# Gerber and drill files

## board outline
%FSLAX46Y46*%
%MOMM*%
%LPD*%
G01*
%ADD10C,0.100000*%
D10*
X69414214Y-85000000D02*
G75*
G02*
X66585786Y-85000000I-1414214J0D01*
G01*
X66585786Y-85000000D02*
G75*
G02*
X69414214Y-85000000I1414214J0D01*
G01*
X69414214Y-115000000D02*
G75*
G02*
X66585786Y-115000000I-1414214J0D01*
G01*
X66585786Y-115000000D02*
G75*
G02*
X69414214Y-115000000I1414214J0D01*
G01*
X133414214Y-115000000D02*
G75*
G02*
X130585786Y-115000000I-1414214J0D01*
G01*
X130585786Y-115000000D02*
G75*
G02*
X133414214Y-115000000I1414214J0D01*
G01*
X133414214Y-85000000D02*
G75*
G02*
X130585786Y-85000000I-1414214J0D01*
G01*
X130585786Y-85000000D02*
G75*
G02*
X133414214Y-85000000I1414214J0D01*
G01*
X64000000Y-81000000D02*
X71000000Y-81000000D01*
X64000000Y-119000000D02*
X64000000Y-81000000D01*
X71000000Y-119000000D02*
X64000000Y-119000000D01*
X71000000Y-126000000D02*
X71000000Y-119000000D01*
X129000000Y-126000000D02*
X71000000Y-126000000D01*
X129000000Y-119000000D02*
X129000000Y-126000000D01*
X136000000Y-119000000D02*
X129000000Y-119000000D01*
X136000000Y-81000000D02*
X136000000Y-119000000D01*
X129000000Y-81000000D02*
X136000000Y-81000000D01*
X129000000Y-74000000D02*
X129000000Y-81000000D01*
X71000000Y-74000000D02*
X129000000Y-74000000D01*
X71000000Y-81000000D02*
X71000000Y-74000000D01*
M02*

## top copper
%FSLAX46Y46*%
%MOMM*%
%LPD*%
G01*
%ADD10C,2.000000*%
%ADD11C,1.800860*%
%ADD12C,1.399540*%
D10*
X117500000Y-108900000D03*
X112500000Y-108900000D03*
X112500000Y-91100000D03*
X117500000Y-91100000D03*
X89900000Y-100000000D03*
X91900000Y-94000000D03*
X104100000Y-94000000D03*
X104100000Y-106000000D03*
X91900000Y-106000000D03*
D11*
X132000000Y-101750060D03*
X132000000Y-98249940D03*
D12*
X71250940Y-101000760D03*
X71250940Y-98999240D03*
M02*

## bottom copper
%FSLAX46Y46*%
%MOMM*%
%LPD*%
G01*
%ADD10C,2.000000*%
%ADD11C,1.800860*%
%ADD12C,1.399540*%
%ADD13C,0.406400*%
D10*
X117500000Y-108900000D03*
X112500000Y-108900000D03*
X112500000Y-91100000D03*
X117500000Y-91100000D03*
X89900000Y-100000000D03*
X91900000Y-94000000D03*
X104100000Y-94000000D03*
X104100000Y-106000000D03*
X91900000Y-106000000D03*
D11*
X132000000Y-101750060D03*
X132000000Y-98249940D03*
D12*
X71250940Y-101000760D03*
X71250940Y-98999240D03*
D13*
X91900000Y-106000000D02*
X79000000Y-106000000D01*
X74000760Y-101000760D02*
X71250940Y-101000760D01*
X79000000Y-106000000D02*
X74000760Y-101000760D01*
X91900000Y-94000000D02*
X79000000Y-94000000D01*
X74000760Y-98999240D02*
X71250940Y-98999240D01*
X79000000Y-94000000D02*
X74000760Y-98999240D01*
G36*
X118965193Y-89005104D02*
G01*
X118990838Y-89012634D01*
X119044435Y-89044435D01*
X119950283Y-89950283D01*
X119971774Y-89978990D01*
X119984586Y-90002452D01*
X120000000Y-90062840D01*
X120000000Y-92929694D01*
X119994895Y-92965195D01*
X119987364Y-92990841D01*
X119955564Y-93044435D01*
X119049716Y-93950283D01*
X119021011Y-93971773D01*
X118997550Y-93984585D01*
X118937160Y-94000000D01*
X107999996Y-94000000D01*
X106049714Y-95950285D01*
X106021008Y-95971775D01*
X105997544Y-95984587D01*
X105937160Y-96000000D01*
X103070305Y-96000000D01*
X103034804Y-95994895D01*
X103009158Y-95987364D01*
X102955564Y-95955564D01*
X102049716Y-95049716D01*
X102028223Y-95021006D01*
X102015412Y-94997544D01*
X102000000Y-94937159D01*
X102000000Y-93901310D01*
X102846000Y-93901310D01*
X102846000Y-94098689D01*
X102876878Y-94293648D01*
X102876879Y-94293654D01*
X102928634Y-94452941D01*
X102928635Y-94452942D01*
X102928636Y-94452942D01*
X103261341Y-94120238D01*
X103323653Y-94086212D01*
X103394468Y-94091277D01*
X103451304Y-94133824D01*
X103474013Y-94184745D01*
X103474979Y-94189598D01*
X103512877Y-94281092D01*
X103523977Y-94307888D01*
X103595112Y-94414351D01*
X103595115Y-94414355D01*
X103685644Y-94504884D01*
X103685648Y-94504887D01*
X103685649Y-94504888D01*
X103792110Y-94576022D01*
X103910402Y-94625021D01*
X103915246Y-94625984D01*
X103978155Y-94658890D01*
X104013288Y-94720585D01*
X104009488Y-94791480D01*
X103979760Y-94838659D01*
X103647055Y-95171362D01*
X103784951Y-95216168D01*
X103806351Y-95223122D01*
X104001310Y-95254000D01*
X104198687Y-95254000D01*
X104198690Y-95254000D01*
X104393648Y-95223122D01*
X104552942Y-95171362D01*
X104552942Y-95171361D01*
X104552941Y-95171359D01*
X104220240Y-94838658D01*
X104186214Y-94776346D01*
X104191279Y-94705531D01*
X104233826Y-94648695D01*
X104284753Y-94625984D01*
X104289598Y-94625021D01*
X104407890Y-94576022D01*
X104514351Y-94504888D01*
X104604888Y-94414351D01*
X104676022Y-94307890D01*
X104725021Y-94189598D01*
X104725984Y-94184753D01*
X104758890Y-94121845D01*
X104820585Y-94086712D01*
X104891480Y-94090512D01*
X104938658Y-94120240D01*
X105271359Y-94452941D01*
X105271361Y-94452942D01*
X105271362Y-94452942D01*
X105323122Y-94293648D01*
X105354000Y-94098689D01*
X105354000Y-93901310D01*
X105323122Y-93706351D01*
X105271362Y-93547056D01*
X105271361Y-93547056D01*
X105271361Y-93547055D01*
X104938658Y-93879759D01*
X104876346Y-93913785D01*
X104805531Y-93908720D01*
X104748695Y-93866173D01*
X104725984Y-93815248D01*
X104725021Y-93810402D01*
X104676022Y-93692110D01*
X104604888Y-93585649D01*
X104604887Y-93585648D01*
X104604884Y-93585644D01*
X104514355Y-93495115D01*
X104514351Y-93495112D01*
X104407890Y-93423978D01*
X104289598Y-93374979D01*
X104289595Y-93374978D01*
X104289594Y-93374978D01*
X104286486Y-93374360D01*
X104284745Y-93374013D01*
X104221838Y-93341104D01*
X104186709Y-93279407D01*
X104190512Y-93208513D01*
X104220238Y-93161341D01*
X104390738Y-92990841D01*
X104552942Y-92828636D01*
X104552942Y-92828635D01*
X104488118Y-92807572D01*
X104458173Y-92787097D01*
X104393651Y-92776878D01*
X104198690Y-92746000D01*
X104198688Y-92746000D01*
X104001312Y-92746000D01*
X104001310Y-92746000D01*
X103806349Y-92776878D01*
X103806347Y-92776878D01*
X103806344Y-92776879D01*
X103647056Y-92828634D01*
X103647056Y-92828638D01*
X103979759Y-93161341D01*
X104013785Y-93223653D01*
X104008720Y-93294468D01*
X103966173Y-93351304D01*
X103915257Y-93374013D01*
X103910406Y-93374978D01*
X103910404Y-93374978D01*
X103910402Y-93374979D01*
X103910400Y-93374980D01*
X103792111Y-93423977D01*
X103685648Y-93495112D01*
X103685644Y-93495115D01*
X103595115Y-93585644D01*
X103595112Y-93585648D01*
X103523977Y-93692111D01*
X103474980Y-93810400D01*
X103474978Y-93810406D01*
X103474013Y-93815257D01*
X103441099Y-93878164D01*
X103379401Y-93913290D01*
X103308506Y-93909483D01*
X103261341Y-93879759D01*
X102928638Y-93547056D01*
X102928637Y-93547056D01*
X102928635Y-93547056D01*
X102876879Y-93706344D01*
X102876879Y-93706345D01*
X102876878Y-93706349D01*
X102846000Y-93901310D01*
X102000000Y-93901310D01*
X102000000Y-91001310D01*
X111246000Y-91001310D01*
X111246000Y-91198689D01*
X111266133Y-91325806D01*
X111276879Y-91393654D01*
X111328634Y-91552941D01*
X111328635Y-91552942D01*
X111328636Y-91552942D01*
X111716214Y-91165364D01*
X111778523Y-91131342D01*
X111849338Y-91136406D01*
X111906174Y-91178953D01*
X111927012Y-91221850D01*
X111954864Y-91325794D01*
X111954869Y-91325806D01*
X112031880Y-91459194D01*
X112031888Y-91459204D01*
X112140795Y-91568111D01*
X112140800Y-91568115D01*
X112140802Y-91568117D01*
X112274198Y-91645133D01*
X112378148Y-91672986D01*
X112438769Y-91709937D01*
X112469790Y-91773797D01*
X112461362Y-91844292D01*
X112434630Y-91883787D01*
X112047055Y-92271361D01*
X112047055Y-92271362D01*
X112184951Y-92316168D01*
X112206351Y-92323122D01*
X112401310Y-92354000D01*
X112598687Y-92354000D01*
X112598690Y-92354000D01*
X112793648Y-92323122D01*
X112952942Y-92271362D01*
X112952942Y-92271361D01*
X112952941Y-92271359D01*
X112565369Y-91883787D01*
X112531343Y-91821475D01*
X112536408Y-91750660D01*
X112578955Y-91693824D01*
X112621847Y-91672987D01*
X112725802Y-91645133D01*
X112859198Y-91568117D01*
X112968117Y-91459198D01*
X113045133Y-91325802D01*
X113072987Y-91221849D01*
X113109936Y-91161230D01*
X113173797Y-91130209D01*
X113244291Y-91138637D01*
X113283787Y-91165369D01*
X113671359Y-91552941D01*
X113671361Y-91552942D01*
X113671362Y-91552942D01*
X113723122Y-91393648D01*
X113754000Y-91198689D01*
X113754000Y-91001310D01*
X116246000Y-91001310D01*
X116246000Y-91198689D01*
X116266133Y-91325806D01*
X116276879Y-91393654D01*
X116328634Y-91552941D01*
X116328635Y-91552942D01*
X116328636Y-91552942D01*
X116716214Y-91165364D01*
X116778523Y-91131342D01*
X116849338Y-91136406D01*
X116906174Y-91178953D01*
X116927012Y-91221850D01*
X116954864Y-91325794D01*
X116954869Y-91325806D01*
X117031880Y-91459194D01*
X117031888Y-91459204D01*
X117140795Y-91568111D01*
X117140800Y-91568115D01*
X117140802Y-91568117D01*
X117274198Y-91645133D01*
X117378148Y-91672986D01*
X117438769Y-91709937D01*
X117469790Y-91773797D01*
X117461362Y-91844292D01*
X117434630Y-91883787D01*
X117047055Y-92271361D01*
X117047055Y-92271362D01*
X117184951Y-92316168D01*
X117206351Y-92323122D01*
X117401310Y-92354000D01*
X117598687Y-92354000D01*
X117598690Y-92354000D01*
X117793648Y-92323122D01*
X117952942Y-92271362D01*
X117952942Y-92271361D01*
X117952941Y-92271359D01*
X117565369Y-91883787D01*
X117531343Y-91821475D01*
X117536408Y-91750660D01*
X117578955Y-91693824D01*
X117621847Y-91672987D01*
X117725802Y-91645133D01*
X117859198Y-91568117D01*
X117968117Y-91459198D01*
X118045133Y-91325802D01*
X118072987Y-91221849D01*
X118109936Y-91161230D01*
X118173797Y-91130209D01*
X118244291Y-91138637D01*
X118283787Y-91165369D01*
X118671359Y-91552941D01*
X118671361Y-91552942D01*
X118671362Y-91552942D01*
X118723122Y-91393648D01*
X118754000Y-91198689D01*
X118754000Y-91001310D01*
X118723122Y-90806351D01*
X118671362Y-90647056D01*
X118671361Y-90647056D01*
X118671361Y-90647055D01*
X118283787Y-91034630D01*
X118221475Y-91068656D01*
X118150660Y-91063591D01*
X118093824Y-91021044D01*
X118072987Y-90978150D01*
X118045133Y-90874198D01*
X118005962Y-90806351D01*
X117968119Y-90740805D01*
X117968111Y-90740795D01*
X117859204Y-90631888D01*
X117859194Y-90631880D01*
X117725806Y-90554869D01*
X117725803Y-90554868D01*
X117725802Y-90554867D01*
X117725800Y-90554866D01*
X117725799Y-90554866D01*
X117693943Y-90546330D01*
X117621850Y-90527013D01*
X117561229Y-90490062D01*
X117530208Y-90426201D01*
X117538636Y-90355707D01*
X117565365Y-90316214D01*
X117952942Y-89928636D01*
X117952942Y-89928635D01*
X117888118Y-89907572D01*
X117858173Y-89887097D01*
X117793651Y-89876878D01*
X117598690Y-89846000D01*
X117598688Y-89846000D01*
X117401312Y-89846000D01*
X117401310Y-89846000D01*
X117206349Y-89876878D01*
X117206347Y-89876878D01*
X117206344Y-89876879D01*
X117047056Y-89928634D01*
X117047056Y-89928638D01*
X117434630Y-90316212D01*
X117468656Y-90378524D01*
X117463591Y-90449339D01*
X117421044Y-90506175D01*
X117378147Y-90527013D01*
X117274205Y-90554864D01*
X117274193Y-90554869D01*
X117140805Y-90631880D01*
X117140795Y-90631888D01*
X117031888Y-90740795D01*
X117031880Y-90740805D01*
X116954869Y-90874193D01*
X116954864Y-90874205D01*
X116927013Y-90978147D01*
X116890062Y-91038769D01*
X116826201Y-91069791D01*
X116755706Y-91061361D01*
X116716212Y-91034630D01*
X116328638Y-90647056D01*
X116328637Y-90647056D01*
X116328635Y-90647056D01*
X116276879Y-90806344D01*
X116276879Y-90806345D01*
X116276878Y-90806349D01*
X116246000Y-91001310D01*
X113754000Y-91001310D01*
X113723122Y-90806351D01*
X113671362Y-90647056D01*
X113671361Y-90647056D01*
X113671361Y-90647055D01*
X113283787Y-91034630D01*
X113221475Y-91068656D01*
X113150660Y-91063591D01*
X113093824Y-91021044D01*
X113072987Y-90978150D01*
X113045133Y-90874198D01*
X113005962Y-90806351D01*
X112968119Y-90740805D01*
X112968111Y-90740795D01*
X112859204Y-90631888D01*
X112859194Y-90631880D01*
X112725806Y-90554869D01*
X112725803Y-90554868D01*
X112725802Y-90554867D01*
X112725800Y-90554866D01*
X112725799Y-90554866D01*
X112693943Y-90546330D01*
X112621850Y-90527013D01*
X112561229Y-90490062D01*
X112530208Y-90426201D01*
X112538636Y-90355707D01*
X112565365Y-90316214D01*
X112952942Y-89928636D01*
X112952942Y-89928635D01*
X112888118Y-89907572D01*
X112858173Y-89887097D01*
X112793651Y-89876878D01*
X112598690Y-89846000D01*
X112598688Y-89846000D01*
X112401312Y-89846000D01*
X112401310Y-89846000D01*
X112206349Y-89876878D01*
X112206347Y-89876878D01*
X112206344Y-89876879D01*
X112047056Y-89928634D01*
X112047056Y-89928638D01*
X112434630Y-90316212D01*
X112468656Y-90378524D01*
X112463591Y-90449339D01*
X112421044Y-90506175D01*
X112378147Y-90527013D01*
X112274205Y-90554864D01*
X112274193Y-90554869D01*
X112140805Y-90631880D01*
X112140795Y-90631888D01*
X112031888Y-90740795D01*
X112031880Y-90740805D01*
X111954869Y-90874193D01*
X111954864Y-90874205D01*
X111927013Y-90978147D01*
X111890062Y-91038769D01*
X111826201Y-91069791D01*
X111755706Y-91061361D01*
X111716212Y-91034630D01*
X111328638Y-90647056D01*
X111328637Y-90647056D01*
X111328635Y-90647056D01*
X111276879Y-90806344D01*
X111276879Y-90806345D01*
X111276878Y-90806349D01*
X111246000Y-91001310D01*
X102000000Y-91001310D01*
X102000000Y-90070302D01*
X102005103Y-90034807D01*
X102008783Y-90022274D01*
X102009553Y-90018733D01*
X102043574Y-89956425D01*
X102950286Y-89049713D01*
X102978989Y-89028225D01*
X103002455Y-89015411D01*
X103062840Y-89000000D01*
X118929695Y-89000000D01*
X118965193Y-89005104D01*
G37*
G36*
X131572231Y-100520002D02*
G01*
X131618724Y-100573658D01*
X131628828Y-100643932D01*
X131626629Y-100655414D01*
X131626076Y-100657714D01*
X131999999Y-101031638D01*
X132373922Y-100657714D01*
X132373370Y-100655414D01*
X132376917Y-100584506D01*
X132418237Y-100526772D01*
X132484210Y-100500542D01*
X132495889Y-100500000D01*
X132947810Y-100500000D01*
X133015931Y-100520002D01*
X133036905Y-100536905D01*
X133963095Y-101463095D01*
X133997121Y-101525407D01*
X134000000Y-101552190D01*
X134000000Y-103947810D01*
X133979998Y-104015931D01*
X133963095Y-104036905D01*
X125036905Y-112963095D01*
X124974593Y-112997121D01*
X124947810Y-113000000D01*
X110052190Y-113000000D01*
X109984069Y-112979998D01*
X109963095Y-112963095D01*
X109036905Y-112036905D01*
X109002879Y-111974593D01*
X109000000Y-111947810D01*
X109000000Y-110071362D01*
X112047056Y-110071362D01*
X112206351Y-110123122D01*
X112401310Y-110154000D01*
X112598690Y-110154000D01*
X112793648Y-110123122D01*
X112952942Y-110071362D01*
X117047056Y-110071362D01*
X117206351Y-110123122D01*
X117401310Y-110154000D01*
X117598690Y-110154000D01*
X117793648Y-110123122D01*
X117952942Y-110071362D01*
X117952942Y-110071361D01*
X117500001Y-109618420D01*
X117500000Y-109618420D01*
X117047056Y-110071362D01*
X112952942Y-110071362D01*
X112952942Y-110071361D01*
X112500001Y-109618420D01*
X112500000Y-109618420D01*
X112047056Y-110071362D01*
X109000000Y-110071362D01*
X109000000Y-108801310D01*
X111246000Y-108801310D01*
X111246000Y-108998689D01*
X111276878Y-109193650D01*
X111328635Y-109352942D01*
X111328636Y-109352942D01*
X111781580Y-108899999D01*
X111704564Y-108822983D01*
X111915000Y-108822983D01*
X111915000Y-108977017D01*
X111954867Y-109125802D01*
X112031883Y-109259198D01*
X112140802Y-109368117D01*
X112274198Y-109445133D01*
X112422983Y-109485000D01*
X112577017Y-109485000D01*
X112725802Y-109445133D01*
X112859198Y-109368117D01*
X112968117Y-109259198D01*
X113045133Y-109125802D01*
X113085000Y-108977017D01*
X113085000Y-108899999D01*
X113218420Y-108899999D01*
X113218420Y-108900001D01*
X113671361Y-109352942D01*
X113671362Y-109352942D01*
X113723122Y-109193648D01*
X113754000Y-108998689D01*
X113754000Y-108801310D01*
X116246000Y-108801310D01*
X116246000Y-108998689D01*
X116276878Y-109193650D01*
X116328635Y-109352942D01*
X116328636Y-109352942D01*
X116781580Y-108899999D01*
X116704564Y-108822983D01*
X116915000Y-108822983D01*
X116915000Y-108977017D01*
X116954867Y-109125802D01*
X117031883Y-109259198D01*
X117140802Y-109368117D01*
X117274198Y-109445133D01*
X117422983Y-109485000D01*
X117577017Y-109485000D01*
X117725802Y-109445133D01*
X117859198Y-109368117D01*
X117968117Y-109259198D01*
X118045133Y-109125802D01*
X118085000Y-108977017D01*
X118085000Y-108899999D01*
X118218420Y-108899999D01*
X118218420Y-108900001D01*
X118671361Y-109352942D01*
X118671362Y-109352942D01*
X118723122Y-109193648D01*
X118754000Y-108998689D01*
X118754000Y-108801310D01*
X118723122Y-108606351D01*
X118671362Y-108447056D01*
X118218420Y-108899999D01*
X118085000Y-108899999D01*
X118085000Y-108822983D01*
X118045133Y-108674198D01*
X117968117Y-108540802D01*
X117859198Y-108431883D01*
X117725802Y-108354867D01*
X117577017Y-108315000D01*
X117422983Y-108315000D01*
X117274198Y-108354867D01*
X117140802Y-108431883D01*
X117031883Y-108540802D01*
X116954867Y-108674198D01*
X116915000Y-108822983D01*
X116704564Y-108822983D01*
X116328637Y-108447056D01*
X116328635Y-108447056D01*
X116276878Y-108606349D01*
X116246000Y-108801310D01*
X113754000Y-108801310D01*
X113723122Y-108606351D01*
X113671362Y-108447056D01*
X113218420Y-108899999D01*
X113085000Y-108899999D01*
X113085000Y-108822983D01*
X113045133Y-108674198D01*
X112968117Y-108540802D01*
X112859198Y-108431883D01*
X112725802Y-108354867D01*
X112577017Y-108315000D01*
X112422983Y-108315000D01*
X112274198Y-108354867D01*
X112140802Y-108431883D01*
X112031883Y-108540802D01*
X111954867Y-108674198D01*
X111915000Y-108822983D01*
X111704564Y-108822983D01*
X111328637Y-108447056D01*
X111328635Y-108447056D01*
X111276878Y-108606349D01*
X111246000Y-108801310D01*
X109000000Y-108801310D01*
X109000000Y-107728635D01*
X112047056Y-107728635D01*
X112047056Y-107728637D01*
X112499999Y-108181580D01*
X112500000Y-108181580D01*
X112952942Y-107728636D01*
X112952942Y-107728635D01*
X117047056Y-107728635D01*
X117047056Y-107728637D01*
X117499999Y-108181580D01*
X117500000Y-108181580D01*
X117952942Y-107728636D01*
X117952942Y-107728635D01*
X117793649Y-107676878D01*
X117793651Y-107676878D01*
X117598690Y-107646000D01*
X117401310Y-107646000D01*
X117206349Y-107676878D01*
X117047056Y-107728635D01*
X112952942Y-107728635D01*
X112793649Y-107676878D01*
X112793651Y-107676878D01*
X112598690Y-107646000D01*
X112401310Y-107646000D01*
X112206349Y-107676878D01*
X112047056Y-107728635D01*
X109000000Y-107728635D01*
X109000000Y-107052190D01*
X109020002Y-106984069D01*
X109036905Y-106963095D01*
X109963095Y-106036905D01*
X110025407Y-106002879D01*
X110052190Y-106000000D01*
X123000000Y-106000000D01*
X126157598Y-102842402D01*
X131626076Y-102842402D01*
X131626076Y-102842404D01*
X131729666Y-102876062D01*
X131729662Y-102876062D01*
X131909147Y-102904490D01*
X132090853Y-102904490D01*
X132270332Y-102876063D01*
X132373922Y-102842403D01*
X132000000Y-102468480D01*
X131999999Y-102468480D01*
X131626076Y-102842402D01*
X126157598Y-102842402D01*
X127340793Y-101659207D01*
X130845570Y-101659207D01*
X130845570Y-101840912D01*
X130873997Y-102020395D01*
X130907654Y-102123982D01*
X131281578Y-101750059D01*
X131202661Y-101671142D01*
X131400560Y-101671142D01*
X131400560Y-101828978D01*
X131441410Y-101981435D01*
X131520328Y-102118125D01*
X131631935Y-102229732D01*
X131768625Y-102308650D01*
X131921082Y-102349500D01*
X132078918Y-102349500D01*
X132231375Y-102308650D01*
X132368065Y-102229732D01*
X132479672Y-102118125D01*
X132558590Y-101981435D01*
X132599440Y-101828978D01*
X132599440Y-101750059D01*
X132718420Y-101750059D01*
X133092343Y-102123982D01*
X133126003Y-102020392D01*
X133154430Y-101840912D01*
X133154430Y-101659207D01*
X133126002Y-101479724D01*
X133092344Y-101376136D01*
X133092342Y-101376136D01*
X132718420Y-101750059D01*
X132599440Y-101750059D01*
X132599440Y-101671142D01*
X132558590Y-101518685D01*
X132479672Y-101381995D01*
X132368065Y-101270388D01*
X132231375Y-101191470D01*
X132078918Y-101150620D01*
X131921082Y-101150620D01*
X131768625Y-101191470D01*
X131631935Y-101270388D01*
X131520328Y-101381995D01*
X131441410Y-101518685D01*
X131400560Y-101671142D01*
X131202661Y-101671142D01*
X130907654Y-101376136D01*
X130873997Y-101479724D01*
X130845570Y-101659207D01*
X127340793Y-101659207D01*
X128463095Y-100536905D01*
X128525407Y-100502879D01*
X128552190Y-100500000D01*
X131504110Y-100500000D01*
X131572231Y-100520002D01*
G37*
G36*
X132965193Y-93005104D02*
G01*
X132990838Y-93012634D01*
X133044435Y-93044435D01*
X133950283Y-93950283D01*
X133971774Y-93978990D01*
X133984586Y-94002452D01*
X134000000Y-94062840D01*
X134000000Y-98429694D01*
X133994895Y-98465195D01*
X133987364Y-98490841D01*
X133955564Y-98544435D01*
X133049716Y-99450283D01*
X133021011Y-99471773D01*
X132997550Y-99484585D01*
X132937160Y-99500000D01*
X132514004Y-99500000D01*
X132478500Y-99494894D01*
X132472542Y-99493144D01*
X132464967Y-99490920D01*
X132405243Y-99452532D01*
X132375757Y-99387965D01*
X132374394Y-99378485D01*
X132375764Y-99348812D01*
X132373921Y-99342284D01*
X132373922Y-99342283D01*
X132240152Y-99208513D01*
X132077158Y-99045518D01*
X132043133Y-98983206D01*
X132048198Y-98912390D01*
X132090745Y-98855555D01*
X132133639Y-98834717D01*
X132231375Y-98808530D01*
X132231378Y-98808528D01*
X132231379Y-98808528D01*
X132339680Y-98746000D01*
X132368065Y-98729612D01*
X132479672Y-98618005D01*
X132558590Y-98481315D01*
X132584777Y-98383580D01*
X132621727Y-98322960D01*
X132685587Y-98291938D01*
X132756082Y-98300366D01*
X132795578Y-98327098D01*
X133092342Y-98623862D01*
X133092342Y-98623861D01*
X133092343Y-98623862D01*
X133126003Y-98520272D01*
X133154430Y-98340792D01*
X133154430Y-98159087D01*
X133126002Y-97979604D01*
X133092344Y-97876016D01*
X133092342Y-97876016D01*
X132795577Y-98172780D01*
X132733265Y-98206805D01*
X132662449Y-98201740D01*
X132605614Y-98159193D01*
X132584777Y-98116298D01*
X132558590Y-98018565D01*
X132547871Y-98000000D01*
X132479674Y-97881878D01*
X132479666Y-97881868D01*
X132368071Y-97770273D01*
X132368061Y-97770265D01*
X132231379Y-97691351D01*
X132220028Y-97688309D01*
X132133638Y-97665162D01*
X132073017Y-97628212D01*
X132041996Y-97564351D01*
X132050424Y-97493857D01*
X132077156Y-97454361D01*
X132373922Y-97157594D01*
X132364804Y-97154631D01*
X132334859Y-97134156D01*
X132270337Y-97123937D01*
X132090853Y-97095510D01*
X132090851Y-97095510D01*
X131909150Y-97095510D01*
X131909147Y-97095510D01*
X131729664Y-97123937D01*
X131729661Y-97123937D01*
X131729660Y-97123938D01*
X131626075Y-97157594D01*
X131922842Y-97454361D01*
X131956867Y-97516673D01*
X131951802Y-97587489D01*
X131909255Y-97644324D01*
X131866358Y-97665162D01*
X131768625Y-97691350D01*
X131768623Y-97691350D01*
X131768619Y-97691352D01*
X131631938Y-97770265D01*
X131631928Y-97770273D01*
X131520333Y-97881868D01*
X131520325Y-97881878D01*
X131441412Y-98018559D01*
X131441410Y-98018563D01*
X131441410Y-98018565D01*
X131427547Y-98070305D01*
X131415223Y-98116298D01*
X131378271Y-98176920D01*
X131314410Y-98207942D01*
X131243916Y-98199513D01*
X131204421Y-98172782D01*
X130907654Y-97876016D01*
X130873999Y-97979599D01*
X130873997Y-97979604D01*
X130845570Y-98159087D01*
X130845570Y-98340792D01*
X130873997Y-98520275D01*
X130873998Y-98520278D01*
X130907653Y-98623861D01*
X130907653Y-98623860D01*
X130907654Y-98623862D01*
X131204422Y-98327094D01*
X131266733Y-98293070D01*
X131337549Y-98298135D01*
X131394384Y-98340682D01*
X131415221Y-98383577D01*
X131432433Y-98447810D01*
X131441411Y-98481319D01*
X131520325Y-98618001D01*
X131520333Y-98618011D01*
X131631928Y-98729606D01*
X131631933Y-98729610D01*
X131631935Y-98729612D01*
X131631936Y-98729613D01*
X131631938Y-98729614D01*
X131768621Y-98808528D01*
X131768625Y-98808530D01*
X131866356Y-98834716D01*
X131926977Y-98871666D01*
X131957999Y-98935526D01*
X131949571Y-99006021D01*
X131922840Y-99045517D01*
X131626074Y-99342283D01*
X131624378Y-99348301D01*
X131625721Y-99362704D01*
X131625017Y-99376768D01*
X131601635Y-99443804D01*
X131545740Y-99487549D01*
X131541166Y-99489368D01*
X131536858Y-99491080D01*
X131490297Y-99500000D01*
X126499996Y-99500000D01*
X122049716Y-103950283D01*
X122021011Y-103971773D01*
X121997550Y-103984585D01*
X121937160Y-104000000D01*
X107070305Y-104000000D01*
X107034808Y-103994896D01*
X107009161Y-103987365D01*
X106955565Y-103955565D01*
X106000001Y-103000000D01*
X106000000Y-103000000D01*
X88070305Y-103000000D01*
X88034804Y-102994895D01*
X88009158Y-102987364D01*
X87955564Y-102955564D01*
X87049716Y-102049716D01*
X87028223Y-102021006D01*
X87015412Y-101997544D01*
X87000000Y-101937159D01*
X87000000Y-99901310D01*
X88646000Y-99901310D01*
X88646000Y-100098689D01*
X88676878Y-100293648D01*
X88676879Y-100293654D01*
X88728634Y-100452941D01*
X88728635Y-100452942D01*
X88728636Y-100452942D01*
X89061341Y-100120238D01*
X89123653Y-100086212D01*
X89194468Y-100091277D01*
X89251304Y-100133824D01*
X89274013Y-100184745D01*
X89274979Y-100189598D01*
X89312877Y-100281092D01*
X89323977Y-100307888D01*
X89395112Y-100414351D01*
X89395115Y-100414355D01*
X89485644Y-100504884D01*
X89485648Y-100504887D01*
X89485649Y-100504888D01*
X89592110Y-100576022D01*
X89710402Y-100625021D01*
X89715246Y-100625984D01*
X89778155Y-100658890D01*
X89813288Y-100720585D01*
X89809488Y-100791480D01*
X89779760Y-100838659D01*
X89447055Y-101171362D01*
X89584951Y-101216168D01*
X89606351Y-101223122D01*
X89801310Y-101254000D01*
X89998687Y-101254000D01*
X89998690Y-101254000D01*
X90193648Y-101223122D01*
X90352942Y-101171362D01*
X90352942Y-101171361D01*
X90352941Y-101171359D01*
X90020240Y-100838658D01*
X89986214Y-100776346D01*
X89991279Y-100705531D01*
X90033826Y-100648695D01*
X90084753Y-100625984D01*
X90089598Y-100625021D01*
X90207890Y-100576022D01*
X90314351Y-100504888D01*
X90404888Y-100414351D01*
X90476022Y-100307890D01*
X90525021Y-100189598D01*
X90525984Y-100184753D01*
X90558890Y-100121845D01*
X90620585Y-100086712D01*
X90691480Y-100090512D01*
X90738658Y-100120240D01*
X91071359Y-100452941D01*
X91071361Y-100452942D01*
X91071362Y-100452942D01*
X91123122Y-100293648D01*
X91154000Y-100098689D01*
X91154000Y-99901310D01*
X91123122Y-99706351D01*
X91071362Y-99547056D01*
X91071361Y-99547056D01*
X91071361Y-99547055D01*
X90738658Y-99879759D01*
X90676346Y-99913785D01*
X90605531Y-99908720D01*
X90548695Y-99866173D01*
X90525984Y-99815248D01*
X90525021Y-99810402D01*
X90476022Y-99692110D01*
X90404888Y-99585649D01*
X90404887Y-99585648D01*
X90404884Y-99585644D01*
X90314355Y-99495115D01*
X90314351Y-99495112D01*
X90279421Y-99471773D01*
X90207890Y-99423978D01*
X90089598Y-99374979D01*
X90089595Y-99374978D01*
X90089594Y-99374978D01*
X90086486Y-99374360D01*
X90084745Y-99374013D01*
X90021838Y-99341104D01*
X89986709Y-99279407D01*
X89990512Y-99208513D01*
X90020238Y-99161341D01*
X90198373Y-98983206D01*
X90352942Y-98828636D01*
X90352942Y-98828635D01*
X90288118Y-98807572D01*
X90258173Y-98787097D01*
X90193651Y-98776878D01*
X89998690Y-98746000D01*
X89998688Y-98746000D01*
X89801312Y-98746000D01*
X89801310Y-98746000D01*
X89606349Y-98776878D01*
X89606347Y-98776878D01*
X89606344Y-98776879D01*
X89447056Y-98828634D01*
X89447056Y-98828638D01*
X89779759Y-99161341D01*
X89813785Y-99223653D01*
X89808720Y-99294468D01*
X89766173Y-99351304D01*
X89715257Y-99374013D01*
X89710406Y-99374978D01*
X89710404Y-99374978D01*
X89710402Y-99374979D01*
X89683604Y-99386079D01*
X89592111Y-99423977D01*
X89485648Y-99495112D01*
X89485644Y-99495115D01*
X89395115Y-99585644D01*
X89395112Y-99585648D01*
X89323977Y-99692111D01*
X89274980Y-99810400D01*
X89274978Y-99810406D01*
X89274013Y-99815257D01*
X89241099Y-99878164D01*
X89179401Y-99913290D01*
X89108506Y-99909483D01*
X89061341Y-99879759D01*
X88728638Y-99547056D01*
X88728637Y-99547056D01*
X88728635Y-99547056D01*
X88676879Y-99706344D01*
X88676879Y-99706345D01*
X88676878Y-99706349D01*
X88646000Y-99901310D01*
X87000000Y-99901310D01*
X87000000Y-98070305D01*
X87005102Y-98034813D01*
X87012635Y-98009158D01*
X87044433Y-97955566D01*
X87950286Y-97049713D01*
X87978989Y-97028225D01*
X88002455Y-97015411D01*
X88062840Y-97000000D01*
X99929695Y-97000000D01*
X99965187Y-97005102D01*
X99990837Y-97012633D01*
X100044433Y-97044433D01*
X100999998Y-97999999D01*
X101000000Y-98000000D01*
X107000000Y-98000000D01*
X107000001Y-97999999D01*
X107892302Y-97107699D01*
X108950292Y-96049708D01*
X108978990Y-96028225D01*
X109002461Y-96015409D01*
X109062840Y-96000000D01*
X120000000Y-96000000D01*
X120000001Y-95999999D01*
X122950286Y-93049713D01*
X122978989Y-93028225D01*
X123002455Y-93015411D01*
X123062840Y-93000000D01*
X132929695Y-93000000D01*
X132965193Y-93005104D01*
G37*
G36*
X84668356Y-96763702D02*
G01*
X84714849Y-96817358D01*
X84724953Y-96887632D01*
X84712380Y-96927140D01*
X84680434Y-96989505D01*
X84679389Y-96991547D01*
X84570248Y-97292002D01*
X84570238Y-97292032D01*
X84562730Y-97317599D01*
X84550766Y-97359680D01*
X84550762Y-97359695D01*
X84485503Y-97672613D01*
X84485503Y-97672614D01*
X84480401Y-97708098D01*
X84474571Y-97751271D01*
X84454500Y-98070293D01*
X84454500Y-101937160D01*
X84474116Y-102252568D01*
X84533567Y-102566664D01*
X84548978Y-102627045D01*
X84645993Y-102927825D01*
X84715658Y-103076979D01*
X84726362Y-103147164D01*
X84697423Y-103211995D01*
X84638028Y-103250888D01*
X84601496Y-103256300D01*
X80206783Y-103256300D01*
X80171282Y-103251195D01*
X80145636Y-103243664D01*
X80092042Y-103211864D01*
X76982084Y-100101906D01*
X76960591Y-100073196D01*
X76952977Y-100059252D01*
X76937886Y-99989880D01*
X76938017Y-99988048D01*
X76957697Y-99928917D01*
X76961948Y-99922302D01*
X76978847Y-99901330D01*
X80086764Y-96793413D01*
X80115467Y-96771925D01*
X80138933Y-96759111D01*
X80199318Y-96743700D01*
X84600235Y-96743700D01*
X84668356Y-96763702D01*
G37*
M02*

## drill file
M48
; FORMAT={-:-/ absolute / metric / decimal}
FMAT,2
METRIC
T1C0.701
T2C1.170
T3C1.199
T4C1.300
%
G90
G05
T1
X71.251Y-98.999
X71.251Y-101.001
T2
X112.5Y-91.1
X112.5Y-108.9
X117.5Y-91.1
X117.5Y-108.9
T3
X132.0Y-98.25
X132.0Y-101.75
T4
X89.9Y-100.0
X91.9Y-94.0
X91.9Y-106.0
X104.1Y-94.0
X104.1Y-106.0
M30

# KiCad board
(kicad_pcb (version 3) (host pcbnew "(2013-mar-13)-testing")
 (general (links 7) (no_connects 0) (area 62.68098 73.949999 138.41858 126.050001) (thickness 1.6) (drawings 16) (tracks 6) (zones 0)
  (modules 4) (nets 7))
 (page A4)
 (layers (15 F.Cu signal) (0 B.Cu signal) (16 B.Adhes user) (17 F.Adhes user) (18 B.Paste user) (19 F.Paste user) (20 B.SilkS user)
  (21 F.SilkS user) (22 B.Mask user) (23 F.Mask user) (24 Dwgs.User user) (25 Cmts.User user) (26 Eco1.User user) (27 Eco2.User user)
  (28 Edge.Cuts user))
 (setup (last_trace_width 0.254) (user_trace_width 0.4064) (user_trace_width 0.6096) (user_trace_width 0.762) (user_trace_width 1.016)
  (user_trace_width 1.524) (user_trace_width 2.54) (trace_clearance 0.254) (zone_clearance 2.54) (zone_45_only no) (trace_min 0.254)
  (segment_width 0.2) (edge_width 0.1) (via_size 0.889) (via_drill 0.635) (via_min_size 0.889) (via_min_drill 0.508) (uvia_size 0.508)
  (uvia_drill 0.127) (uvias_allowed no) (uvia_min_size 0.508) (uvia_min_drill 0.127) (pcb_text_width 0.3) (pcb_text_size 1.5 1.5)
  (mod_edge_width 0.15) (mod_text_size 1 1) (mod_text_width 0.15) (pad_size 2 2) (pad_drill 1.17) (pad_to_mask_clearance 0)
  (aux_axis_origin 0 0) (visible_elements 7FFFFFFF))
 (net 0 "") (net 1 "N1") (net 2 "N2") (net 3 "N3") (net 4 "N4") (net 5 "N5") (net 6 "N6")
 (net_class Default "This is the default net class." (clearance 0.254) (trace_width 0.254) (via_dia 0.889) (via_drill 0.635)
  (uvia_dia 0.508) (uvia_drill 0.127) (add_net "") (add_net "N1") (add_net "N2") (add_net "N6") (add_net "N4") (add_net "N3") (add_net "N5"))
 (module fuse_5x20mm (layer F.Cu) (at 115 100 270)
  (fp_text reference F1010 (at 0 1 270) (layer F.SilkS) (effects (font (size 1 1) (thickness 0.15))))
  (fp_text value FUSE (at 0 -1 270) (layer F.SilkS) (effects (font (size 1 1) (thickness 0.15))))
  (pad 2 thru_hole circle (at 8.9 -2.5 270) (size 2 2) (drill 1.17) (layers *.Cu *.Mask F.SilkS) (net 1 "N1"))
  (pad 2 thru_hole circle (at 8.9 2.5 270) (size 2 2) (drill 1.17) (layers *.Cu *.Mask F.SilkS) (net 1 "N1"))
  (pad 1 thru_hole circle (at -8.9 2.5 270) (size 2 2) (drill 1.17) (layers *.Cu *.Mask F.SilkS) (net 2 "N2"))
  (pad 1 thru_hole circle (at -8.9 -2.5 270) (size 2 2) (drill 1.17) (layers *.Cu *.Mask F.SilkS) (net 2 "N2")))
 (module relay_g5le (layer F.Cu) (at 98 100)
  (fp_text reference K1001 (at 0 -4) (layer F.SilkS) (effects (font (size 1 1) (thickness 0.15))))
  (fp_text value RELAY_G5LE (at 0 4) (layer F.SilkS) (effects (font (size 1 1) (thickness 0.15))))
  (pad 1 thru_hole circle (at -8.1 0) (size 2 2) (drill 1.3) (layers *.Cu *.Mask F.SilkS) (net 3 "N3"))
  (pad 2 thru_hole circle (at -6.1 -6) (size 2 2) (drill 1.3) (layers *.Cu *.Mask F.SilkS) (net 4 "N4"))
  (pad 3 thru_hole circle (at 6.1 -6) (size 2 2) (drill 1.3) (layers *.Cu *.Mask F.SilkS) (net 2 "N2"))
  (pad 4 thru_hole circle (at 6.1 6) (size 2 2) (drill 1.3) (layers *.Cu *.Mask F.SilkS) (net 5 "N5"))
  (pad 5 thru_hole circle (at -6.1 6) (size 2 2) (drill 1.3) (layers *.Cu *.Mask F.SilkS) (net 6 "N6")))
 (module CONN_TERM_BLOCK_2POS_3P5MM (layer F.Cu) (at 132 100 270)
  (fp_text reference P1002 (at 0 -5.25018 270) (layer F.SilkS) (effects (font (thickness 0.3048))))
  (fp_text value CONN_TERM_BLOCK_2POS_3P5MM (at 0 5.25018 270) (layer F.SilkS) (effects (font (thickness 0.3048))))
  (pad 1 thru_hole circle (at 1.75006 0 270) (size 1.80086 1.80086) (drill 1.19888) (layers *.Cu *.Mask F.SilkS) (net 1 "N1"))
  (pad 2 thru_hole circle (at -1.75006 0 270) (size 1.80086 1.80086) (drill 1.19888) (layers *.Cu *.Mask F.SilkS) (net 3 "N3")))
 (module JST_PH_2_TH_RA (layer F.Cu) (at 65 100 90)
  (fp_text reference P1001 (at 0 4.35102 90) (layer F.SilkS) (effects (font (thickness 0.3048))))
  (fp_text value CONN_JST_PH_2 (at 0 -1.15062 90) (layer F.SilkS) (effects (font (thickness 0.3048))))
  (pad 2 thru_hole circle (at -1.00076 6.25094 90) (size 1.39954 1.39954) (drill 0.70104) (layers *.Cu *.Mask F.SilkS) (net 6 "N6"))
  (pad 1 thru_hole circle (at 1.00076 6.25094 90) (size 1.39954 1.39954) (drill 0.70104) (layers *.Cu *.Mask F.SilkS) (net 4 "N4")))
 (gr_circle (center 68 85) (end 69 86) (layer Edge.Cuts) (width 0.1))
 (gr_circle (center 68 115) (end 69 116) (layer Edge.Cuts) (width 0.1))
 (gr_circle (center 132 115) (end 133 116) (layer Edge.Cuts) (width 0.1))
 (gr_circle (center 132 85) (end 131 84) (layer Edge.Cuts) (width 0.1))
 (gr_line (start 64 81) (end 71 81) (angle 90) (layer Edge.Cuts) (width 0.1))
 (gr_line (start 64 119) (end 64 81) (angle 90) (layer Edge.Cuts) (width 0.1))
 (gr_line (start 71 119) (end 64 119) (angle 90) (layer Edge.Cuts) (width 0.1))
 (gr_line (start 71 126) (end 71 119) (angle 90) (layer Edge.Cuts) (width 0.1))
 (gr_line (start 129 126) (end 71 126) (angle 90) (layer Edge.Cuts) (width 0.1))
 (gr_line (start 129 119) (end 129 126) (angle 90) (layer Edge.Cuts) (width 0.1))
 (gr_line (start 136 119) (end 129 119) (angle 90) (layer Edge.Cuts) (width 0.1))
 (gr_line (start 136 81) (end 136 119) (angle 90) (layer Edge.Cuts) (width 0.1))
 (gr_line (start 129 81) (end 136 81) (angle 90) (layer Edge.Cuts) (width 0.1))
 (gr_line (start 129 74) (end 129 81) (angle 90) (layer Edge.Cuts) (width 0.1))
 (gr_line (start 71 74) (end 129 74) (angle 90) (layer Edge.Cuts) (width 0.1))
 (gr_line (start 71 81) (end 71 74) (angle 90) (layer Edge.Cuts) (width 0.1))
 (segment (start 91.9 106) (end 79 106) (width 0.4064) (layer B.Cu) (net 6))
 (segment (start 74.00076 101.00076) (end 71.25094 101.00076) (width 0.4064) (layer B.Cu) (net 6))
 (segment (start 79 106) (end 74.00076 101.00076) (width 0.4064) (layer B.Cu) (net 6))
 (segment (start 91.9 94) (end 79 94) (width 0.4064) (layer B.Cu) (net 4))
 (segment (start 74.00076 98.99924) (end 71.25094 98.99924) (width 0.4064) (layer B.Cu) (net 4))
 (segment (start 79 94) (end 74.00076 98.99924) (width 0.4064) (layer B.Cu) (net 4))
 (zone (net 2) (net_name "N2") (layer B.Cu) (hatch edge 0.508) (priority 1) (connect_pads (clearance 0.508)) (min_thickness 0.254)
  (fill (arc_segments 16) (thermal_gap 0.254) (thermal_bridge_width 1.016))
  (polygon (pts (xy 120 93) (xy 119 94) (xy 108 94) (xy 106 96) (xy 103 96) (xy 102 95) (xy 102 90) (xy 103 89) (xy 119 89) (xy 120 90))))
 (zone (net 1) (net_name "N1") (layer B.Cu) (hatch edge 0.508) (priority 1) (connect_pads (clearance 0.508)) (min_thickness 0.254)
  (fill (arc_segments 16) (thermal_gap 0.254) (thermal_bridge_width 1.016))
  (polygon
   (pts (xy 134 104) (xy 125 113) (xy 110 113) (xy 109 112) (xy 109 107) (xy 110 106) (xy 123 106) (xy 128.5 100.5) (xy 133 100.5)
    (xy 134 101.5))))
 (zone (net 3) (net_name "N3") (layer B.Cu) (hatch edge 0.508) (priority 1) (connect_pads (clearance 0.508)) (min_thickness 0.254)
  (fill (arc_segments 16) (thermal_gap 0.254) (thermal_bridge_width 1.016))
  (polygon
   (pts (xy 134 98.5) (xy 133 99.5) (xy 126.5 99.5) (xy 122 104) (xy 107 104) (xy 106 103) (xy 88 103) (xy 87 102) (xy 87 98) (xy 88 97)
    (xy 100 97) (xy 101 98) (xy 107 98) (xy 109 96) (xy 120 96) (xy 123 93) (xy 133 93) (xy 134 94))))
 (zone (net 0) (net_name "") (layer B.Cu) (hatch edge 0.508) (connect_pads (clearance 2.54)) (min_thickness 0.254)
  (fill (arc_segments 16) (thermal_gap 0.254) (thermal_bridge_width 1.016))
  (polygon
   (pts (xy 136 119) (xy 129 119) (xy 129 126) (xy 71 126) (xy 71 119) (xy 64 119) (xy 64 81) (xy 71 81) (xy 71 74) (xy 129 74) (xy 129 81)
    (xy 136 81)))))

